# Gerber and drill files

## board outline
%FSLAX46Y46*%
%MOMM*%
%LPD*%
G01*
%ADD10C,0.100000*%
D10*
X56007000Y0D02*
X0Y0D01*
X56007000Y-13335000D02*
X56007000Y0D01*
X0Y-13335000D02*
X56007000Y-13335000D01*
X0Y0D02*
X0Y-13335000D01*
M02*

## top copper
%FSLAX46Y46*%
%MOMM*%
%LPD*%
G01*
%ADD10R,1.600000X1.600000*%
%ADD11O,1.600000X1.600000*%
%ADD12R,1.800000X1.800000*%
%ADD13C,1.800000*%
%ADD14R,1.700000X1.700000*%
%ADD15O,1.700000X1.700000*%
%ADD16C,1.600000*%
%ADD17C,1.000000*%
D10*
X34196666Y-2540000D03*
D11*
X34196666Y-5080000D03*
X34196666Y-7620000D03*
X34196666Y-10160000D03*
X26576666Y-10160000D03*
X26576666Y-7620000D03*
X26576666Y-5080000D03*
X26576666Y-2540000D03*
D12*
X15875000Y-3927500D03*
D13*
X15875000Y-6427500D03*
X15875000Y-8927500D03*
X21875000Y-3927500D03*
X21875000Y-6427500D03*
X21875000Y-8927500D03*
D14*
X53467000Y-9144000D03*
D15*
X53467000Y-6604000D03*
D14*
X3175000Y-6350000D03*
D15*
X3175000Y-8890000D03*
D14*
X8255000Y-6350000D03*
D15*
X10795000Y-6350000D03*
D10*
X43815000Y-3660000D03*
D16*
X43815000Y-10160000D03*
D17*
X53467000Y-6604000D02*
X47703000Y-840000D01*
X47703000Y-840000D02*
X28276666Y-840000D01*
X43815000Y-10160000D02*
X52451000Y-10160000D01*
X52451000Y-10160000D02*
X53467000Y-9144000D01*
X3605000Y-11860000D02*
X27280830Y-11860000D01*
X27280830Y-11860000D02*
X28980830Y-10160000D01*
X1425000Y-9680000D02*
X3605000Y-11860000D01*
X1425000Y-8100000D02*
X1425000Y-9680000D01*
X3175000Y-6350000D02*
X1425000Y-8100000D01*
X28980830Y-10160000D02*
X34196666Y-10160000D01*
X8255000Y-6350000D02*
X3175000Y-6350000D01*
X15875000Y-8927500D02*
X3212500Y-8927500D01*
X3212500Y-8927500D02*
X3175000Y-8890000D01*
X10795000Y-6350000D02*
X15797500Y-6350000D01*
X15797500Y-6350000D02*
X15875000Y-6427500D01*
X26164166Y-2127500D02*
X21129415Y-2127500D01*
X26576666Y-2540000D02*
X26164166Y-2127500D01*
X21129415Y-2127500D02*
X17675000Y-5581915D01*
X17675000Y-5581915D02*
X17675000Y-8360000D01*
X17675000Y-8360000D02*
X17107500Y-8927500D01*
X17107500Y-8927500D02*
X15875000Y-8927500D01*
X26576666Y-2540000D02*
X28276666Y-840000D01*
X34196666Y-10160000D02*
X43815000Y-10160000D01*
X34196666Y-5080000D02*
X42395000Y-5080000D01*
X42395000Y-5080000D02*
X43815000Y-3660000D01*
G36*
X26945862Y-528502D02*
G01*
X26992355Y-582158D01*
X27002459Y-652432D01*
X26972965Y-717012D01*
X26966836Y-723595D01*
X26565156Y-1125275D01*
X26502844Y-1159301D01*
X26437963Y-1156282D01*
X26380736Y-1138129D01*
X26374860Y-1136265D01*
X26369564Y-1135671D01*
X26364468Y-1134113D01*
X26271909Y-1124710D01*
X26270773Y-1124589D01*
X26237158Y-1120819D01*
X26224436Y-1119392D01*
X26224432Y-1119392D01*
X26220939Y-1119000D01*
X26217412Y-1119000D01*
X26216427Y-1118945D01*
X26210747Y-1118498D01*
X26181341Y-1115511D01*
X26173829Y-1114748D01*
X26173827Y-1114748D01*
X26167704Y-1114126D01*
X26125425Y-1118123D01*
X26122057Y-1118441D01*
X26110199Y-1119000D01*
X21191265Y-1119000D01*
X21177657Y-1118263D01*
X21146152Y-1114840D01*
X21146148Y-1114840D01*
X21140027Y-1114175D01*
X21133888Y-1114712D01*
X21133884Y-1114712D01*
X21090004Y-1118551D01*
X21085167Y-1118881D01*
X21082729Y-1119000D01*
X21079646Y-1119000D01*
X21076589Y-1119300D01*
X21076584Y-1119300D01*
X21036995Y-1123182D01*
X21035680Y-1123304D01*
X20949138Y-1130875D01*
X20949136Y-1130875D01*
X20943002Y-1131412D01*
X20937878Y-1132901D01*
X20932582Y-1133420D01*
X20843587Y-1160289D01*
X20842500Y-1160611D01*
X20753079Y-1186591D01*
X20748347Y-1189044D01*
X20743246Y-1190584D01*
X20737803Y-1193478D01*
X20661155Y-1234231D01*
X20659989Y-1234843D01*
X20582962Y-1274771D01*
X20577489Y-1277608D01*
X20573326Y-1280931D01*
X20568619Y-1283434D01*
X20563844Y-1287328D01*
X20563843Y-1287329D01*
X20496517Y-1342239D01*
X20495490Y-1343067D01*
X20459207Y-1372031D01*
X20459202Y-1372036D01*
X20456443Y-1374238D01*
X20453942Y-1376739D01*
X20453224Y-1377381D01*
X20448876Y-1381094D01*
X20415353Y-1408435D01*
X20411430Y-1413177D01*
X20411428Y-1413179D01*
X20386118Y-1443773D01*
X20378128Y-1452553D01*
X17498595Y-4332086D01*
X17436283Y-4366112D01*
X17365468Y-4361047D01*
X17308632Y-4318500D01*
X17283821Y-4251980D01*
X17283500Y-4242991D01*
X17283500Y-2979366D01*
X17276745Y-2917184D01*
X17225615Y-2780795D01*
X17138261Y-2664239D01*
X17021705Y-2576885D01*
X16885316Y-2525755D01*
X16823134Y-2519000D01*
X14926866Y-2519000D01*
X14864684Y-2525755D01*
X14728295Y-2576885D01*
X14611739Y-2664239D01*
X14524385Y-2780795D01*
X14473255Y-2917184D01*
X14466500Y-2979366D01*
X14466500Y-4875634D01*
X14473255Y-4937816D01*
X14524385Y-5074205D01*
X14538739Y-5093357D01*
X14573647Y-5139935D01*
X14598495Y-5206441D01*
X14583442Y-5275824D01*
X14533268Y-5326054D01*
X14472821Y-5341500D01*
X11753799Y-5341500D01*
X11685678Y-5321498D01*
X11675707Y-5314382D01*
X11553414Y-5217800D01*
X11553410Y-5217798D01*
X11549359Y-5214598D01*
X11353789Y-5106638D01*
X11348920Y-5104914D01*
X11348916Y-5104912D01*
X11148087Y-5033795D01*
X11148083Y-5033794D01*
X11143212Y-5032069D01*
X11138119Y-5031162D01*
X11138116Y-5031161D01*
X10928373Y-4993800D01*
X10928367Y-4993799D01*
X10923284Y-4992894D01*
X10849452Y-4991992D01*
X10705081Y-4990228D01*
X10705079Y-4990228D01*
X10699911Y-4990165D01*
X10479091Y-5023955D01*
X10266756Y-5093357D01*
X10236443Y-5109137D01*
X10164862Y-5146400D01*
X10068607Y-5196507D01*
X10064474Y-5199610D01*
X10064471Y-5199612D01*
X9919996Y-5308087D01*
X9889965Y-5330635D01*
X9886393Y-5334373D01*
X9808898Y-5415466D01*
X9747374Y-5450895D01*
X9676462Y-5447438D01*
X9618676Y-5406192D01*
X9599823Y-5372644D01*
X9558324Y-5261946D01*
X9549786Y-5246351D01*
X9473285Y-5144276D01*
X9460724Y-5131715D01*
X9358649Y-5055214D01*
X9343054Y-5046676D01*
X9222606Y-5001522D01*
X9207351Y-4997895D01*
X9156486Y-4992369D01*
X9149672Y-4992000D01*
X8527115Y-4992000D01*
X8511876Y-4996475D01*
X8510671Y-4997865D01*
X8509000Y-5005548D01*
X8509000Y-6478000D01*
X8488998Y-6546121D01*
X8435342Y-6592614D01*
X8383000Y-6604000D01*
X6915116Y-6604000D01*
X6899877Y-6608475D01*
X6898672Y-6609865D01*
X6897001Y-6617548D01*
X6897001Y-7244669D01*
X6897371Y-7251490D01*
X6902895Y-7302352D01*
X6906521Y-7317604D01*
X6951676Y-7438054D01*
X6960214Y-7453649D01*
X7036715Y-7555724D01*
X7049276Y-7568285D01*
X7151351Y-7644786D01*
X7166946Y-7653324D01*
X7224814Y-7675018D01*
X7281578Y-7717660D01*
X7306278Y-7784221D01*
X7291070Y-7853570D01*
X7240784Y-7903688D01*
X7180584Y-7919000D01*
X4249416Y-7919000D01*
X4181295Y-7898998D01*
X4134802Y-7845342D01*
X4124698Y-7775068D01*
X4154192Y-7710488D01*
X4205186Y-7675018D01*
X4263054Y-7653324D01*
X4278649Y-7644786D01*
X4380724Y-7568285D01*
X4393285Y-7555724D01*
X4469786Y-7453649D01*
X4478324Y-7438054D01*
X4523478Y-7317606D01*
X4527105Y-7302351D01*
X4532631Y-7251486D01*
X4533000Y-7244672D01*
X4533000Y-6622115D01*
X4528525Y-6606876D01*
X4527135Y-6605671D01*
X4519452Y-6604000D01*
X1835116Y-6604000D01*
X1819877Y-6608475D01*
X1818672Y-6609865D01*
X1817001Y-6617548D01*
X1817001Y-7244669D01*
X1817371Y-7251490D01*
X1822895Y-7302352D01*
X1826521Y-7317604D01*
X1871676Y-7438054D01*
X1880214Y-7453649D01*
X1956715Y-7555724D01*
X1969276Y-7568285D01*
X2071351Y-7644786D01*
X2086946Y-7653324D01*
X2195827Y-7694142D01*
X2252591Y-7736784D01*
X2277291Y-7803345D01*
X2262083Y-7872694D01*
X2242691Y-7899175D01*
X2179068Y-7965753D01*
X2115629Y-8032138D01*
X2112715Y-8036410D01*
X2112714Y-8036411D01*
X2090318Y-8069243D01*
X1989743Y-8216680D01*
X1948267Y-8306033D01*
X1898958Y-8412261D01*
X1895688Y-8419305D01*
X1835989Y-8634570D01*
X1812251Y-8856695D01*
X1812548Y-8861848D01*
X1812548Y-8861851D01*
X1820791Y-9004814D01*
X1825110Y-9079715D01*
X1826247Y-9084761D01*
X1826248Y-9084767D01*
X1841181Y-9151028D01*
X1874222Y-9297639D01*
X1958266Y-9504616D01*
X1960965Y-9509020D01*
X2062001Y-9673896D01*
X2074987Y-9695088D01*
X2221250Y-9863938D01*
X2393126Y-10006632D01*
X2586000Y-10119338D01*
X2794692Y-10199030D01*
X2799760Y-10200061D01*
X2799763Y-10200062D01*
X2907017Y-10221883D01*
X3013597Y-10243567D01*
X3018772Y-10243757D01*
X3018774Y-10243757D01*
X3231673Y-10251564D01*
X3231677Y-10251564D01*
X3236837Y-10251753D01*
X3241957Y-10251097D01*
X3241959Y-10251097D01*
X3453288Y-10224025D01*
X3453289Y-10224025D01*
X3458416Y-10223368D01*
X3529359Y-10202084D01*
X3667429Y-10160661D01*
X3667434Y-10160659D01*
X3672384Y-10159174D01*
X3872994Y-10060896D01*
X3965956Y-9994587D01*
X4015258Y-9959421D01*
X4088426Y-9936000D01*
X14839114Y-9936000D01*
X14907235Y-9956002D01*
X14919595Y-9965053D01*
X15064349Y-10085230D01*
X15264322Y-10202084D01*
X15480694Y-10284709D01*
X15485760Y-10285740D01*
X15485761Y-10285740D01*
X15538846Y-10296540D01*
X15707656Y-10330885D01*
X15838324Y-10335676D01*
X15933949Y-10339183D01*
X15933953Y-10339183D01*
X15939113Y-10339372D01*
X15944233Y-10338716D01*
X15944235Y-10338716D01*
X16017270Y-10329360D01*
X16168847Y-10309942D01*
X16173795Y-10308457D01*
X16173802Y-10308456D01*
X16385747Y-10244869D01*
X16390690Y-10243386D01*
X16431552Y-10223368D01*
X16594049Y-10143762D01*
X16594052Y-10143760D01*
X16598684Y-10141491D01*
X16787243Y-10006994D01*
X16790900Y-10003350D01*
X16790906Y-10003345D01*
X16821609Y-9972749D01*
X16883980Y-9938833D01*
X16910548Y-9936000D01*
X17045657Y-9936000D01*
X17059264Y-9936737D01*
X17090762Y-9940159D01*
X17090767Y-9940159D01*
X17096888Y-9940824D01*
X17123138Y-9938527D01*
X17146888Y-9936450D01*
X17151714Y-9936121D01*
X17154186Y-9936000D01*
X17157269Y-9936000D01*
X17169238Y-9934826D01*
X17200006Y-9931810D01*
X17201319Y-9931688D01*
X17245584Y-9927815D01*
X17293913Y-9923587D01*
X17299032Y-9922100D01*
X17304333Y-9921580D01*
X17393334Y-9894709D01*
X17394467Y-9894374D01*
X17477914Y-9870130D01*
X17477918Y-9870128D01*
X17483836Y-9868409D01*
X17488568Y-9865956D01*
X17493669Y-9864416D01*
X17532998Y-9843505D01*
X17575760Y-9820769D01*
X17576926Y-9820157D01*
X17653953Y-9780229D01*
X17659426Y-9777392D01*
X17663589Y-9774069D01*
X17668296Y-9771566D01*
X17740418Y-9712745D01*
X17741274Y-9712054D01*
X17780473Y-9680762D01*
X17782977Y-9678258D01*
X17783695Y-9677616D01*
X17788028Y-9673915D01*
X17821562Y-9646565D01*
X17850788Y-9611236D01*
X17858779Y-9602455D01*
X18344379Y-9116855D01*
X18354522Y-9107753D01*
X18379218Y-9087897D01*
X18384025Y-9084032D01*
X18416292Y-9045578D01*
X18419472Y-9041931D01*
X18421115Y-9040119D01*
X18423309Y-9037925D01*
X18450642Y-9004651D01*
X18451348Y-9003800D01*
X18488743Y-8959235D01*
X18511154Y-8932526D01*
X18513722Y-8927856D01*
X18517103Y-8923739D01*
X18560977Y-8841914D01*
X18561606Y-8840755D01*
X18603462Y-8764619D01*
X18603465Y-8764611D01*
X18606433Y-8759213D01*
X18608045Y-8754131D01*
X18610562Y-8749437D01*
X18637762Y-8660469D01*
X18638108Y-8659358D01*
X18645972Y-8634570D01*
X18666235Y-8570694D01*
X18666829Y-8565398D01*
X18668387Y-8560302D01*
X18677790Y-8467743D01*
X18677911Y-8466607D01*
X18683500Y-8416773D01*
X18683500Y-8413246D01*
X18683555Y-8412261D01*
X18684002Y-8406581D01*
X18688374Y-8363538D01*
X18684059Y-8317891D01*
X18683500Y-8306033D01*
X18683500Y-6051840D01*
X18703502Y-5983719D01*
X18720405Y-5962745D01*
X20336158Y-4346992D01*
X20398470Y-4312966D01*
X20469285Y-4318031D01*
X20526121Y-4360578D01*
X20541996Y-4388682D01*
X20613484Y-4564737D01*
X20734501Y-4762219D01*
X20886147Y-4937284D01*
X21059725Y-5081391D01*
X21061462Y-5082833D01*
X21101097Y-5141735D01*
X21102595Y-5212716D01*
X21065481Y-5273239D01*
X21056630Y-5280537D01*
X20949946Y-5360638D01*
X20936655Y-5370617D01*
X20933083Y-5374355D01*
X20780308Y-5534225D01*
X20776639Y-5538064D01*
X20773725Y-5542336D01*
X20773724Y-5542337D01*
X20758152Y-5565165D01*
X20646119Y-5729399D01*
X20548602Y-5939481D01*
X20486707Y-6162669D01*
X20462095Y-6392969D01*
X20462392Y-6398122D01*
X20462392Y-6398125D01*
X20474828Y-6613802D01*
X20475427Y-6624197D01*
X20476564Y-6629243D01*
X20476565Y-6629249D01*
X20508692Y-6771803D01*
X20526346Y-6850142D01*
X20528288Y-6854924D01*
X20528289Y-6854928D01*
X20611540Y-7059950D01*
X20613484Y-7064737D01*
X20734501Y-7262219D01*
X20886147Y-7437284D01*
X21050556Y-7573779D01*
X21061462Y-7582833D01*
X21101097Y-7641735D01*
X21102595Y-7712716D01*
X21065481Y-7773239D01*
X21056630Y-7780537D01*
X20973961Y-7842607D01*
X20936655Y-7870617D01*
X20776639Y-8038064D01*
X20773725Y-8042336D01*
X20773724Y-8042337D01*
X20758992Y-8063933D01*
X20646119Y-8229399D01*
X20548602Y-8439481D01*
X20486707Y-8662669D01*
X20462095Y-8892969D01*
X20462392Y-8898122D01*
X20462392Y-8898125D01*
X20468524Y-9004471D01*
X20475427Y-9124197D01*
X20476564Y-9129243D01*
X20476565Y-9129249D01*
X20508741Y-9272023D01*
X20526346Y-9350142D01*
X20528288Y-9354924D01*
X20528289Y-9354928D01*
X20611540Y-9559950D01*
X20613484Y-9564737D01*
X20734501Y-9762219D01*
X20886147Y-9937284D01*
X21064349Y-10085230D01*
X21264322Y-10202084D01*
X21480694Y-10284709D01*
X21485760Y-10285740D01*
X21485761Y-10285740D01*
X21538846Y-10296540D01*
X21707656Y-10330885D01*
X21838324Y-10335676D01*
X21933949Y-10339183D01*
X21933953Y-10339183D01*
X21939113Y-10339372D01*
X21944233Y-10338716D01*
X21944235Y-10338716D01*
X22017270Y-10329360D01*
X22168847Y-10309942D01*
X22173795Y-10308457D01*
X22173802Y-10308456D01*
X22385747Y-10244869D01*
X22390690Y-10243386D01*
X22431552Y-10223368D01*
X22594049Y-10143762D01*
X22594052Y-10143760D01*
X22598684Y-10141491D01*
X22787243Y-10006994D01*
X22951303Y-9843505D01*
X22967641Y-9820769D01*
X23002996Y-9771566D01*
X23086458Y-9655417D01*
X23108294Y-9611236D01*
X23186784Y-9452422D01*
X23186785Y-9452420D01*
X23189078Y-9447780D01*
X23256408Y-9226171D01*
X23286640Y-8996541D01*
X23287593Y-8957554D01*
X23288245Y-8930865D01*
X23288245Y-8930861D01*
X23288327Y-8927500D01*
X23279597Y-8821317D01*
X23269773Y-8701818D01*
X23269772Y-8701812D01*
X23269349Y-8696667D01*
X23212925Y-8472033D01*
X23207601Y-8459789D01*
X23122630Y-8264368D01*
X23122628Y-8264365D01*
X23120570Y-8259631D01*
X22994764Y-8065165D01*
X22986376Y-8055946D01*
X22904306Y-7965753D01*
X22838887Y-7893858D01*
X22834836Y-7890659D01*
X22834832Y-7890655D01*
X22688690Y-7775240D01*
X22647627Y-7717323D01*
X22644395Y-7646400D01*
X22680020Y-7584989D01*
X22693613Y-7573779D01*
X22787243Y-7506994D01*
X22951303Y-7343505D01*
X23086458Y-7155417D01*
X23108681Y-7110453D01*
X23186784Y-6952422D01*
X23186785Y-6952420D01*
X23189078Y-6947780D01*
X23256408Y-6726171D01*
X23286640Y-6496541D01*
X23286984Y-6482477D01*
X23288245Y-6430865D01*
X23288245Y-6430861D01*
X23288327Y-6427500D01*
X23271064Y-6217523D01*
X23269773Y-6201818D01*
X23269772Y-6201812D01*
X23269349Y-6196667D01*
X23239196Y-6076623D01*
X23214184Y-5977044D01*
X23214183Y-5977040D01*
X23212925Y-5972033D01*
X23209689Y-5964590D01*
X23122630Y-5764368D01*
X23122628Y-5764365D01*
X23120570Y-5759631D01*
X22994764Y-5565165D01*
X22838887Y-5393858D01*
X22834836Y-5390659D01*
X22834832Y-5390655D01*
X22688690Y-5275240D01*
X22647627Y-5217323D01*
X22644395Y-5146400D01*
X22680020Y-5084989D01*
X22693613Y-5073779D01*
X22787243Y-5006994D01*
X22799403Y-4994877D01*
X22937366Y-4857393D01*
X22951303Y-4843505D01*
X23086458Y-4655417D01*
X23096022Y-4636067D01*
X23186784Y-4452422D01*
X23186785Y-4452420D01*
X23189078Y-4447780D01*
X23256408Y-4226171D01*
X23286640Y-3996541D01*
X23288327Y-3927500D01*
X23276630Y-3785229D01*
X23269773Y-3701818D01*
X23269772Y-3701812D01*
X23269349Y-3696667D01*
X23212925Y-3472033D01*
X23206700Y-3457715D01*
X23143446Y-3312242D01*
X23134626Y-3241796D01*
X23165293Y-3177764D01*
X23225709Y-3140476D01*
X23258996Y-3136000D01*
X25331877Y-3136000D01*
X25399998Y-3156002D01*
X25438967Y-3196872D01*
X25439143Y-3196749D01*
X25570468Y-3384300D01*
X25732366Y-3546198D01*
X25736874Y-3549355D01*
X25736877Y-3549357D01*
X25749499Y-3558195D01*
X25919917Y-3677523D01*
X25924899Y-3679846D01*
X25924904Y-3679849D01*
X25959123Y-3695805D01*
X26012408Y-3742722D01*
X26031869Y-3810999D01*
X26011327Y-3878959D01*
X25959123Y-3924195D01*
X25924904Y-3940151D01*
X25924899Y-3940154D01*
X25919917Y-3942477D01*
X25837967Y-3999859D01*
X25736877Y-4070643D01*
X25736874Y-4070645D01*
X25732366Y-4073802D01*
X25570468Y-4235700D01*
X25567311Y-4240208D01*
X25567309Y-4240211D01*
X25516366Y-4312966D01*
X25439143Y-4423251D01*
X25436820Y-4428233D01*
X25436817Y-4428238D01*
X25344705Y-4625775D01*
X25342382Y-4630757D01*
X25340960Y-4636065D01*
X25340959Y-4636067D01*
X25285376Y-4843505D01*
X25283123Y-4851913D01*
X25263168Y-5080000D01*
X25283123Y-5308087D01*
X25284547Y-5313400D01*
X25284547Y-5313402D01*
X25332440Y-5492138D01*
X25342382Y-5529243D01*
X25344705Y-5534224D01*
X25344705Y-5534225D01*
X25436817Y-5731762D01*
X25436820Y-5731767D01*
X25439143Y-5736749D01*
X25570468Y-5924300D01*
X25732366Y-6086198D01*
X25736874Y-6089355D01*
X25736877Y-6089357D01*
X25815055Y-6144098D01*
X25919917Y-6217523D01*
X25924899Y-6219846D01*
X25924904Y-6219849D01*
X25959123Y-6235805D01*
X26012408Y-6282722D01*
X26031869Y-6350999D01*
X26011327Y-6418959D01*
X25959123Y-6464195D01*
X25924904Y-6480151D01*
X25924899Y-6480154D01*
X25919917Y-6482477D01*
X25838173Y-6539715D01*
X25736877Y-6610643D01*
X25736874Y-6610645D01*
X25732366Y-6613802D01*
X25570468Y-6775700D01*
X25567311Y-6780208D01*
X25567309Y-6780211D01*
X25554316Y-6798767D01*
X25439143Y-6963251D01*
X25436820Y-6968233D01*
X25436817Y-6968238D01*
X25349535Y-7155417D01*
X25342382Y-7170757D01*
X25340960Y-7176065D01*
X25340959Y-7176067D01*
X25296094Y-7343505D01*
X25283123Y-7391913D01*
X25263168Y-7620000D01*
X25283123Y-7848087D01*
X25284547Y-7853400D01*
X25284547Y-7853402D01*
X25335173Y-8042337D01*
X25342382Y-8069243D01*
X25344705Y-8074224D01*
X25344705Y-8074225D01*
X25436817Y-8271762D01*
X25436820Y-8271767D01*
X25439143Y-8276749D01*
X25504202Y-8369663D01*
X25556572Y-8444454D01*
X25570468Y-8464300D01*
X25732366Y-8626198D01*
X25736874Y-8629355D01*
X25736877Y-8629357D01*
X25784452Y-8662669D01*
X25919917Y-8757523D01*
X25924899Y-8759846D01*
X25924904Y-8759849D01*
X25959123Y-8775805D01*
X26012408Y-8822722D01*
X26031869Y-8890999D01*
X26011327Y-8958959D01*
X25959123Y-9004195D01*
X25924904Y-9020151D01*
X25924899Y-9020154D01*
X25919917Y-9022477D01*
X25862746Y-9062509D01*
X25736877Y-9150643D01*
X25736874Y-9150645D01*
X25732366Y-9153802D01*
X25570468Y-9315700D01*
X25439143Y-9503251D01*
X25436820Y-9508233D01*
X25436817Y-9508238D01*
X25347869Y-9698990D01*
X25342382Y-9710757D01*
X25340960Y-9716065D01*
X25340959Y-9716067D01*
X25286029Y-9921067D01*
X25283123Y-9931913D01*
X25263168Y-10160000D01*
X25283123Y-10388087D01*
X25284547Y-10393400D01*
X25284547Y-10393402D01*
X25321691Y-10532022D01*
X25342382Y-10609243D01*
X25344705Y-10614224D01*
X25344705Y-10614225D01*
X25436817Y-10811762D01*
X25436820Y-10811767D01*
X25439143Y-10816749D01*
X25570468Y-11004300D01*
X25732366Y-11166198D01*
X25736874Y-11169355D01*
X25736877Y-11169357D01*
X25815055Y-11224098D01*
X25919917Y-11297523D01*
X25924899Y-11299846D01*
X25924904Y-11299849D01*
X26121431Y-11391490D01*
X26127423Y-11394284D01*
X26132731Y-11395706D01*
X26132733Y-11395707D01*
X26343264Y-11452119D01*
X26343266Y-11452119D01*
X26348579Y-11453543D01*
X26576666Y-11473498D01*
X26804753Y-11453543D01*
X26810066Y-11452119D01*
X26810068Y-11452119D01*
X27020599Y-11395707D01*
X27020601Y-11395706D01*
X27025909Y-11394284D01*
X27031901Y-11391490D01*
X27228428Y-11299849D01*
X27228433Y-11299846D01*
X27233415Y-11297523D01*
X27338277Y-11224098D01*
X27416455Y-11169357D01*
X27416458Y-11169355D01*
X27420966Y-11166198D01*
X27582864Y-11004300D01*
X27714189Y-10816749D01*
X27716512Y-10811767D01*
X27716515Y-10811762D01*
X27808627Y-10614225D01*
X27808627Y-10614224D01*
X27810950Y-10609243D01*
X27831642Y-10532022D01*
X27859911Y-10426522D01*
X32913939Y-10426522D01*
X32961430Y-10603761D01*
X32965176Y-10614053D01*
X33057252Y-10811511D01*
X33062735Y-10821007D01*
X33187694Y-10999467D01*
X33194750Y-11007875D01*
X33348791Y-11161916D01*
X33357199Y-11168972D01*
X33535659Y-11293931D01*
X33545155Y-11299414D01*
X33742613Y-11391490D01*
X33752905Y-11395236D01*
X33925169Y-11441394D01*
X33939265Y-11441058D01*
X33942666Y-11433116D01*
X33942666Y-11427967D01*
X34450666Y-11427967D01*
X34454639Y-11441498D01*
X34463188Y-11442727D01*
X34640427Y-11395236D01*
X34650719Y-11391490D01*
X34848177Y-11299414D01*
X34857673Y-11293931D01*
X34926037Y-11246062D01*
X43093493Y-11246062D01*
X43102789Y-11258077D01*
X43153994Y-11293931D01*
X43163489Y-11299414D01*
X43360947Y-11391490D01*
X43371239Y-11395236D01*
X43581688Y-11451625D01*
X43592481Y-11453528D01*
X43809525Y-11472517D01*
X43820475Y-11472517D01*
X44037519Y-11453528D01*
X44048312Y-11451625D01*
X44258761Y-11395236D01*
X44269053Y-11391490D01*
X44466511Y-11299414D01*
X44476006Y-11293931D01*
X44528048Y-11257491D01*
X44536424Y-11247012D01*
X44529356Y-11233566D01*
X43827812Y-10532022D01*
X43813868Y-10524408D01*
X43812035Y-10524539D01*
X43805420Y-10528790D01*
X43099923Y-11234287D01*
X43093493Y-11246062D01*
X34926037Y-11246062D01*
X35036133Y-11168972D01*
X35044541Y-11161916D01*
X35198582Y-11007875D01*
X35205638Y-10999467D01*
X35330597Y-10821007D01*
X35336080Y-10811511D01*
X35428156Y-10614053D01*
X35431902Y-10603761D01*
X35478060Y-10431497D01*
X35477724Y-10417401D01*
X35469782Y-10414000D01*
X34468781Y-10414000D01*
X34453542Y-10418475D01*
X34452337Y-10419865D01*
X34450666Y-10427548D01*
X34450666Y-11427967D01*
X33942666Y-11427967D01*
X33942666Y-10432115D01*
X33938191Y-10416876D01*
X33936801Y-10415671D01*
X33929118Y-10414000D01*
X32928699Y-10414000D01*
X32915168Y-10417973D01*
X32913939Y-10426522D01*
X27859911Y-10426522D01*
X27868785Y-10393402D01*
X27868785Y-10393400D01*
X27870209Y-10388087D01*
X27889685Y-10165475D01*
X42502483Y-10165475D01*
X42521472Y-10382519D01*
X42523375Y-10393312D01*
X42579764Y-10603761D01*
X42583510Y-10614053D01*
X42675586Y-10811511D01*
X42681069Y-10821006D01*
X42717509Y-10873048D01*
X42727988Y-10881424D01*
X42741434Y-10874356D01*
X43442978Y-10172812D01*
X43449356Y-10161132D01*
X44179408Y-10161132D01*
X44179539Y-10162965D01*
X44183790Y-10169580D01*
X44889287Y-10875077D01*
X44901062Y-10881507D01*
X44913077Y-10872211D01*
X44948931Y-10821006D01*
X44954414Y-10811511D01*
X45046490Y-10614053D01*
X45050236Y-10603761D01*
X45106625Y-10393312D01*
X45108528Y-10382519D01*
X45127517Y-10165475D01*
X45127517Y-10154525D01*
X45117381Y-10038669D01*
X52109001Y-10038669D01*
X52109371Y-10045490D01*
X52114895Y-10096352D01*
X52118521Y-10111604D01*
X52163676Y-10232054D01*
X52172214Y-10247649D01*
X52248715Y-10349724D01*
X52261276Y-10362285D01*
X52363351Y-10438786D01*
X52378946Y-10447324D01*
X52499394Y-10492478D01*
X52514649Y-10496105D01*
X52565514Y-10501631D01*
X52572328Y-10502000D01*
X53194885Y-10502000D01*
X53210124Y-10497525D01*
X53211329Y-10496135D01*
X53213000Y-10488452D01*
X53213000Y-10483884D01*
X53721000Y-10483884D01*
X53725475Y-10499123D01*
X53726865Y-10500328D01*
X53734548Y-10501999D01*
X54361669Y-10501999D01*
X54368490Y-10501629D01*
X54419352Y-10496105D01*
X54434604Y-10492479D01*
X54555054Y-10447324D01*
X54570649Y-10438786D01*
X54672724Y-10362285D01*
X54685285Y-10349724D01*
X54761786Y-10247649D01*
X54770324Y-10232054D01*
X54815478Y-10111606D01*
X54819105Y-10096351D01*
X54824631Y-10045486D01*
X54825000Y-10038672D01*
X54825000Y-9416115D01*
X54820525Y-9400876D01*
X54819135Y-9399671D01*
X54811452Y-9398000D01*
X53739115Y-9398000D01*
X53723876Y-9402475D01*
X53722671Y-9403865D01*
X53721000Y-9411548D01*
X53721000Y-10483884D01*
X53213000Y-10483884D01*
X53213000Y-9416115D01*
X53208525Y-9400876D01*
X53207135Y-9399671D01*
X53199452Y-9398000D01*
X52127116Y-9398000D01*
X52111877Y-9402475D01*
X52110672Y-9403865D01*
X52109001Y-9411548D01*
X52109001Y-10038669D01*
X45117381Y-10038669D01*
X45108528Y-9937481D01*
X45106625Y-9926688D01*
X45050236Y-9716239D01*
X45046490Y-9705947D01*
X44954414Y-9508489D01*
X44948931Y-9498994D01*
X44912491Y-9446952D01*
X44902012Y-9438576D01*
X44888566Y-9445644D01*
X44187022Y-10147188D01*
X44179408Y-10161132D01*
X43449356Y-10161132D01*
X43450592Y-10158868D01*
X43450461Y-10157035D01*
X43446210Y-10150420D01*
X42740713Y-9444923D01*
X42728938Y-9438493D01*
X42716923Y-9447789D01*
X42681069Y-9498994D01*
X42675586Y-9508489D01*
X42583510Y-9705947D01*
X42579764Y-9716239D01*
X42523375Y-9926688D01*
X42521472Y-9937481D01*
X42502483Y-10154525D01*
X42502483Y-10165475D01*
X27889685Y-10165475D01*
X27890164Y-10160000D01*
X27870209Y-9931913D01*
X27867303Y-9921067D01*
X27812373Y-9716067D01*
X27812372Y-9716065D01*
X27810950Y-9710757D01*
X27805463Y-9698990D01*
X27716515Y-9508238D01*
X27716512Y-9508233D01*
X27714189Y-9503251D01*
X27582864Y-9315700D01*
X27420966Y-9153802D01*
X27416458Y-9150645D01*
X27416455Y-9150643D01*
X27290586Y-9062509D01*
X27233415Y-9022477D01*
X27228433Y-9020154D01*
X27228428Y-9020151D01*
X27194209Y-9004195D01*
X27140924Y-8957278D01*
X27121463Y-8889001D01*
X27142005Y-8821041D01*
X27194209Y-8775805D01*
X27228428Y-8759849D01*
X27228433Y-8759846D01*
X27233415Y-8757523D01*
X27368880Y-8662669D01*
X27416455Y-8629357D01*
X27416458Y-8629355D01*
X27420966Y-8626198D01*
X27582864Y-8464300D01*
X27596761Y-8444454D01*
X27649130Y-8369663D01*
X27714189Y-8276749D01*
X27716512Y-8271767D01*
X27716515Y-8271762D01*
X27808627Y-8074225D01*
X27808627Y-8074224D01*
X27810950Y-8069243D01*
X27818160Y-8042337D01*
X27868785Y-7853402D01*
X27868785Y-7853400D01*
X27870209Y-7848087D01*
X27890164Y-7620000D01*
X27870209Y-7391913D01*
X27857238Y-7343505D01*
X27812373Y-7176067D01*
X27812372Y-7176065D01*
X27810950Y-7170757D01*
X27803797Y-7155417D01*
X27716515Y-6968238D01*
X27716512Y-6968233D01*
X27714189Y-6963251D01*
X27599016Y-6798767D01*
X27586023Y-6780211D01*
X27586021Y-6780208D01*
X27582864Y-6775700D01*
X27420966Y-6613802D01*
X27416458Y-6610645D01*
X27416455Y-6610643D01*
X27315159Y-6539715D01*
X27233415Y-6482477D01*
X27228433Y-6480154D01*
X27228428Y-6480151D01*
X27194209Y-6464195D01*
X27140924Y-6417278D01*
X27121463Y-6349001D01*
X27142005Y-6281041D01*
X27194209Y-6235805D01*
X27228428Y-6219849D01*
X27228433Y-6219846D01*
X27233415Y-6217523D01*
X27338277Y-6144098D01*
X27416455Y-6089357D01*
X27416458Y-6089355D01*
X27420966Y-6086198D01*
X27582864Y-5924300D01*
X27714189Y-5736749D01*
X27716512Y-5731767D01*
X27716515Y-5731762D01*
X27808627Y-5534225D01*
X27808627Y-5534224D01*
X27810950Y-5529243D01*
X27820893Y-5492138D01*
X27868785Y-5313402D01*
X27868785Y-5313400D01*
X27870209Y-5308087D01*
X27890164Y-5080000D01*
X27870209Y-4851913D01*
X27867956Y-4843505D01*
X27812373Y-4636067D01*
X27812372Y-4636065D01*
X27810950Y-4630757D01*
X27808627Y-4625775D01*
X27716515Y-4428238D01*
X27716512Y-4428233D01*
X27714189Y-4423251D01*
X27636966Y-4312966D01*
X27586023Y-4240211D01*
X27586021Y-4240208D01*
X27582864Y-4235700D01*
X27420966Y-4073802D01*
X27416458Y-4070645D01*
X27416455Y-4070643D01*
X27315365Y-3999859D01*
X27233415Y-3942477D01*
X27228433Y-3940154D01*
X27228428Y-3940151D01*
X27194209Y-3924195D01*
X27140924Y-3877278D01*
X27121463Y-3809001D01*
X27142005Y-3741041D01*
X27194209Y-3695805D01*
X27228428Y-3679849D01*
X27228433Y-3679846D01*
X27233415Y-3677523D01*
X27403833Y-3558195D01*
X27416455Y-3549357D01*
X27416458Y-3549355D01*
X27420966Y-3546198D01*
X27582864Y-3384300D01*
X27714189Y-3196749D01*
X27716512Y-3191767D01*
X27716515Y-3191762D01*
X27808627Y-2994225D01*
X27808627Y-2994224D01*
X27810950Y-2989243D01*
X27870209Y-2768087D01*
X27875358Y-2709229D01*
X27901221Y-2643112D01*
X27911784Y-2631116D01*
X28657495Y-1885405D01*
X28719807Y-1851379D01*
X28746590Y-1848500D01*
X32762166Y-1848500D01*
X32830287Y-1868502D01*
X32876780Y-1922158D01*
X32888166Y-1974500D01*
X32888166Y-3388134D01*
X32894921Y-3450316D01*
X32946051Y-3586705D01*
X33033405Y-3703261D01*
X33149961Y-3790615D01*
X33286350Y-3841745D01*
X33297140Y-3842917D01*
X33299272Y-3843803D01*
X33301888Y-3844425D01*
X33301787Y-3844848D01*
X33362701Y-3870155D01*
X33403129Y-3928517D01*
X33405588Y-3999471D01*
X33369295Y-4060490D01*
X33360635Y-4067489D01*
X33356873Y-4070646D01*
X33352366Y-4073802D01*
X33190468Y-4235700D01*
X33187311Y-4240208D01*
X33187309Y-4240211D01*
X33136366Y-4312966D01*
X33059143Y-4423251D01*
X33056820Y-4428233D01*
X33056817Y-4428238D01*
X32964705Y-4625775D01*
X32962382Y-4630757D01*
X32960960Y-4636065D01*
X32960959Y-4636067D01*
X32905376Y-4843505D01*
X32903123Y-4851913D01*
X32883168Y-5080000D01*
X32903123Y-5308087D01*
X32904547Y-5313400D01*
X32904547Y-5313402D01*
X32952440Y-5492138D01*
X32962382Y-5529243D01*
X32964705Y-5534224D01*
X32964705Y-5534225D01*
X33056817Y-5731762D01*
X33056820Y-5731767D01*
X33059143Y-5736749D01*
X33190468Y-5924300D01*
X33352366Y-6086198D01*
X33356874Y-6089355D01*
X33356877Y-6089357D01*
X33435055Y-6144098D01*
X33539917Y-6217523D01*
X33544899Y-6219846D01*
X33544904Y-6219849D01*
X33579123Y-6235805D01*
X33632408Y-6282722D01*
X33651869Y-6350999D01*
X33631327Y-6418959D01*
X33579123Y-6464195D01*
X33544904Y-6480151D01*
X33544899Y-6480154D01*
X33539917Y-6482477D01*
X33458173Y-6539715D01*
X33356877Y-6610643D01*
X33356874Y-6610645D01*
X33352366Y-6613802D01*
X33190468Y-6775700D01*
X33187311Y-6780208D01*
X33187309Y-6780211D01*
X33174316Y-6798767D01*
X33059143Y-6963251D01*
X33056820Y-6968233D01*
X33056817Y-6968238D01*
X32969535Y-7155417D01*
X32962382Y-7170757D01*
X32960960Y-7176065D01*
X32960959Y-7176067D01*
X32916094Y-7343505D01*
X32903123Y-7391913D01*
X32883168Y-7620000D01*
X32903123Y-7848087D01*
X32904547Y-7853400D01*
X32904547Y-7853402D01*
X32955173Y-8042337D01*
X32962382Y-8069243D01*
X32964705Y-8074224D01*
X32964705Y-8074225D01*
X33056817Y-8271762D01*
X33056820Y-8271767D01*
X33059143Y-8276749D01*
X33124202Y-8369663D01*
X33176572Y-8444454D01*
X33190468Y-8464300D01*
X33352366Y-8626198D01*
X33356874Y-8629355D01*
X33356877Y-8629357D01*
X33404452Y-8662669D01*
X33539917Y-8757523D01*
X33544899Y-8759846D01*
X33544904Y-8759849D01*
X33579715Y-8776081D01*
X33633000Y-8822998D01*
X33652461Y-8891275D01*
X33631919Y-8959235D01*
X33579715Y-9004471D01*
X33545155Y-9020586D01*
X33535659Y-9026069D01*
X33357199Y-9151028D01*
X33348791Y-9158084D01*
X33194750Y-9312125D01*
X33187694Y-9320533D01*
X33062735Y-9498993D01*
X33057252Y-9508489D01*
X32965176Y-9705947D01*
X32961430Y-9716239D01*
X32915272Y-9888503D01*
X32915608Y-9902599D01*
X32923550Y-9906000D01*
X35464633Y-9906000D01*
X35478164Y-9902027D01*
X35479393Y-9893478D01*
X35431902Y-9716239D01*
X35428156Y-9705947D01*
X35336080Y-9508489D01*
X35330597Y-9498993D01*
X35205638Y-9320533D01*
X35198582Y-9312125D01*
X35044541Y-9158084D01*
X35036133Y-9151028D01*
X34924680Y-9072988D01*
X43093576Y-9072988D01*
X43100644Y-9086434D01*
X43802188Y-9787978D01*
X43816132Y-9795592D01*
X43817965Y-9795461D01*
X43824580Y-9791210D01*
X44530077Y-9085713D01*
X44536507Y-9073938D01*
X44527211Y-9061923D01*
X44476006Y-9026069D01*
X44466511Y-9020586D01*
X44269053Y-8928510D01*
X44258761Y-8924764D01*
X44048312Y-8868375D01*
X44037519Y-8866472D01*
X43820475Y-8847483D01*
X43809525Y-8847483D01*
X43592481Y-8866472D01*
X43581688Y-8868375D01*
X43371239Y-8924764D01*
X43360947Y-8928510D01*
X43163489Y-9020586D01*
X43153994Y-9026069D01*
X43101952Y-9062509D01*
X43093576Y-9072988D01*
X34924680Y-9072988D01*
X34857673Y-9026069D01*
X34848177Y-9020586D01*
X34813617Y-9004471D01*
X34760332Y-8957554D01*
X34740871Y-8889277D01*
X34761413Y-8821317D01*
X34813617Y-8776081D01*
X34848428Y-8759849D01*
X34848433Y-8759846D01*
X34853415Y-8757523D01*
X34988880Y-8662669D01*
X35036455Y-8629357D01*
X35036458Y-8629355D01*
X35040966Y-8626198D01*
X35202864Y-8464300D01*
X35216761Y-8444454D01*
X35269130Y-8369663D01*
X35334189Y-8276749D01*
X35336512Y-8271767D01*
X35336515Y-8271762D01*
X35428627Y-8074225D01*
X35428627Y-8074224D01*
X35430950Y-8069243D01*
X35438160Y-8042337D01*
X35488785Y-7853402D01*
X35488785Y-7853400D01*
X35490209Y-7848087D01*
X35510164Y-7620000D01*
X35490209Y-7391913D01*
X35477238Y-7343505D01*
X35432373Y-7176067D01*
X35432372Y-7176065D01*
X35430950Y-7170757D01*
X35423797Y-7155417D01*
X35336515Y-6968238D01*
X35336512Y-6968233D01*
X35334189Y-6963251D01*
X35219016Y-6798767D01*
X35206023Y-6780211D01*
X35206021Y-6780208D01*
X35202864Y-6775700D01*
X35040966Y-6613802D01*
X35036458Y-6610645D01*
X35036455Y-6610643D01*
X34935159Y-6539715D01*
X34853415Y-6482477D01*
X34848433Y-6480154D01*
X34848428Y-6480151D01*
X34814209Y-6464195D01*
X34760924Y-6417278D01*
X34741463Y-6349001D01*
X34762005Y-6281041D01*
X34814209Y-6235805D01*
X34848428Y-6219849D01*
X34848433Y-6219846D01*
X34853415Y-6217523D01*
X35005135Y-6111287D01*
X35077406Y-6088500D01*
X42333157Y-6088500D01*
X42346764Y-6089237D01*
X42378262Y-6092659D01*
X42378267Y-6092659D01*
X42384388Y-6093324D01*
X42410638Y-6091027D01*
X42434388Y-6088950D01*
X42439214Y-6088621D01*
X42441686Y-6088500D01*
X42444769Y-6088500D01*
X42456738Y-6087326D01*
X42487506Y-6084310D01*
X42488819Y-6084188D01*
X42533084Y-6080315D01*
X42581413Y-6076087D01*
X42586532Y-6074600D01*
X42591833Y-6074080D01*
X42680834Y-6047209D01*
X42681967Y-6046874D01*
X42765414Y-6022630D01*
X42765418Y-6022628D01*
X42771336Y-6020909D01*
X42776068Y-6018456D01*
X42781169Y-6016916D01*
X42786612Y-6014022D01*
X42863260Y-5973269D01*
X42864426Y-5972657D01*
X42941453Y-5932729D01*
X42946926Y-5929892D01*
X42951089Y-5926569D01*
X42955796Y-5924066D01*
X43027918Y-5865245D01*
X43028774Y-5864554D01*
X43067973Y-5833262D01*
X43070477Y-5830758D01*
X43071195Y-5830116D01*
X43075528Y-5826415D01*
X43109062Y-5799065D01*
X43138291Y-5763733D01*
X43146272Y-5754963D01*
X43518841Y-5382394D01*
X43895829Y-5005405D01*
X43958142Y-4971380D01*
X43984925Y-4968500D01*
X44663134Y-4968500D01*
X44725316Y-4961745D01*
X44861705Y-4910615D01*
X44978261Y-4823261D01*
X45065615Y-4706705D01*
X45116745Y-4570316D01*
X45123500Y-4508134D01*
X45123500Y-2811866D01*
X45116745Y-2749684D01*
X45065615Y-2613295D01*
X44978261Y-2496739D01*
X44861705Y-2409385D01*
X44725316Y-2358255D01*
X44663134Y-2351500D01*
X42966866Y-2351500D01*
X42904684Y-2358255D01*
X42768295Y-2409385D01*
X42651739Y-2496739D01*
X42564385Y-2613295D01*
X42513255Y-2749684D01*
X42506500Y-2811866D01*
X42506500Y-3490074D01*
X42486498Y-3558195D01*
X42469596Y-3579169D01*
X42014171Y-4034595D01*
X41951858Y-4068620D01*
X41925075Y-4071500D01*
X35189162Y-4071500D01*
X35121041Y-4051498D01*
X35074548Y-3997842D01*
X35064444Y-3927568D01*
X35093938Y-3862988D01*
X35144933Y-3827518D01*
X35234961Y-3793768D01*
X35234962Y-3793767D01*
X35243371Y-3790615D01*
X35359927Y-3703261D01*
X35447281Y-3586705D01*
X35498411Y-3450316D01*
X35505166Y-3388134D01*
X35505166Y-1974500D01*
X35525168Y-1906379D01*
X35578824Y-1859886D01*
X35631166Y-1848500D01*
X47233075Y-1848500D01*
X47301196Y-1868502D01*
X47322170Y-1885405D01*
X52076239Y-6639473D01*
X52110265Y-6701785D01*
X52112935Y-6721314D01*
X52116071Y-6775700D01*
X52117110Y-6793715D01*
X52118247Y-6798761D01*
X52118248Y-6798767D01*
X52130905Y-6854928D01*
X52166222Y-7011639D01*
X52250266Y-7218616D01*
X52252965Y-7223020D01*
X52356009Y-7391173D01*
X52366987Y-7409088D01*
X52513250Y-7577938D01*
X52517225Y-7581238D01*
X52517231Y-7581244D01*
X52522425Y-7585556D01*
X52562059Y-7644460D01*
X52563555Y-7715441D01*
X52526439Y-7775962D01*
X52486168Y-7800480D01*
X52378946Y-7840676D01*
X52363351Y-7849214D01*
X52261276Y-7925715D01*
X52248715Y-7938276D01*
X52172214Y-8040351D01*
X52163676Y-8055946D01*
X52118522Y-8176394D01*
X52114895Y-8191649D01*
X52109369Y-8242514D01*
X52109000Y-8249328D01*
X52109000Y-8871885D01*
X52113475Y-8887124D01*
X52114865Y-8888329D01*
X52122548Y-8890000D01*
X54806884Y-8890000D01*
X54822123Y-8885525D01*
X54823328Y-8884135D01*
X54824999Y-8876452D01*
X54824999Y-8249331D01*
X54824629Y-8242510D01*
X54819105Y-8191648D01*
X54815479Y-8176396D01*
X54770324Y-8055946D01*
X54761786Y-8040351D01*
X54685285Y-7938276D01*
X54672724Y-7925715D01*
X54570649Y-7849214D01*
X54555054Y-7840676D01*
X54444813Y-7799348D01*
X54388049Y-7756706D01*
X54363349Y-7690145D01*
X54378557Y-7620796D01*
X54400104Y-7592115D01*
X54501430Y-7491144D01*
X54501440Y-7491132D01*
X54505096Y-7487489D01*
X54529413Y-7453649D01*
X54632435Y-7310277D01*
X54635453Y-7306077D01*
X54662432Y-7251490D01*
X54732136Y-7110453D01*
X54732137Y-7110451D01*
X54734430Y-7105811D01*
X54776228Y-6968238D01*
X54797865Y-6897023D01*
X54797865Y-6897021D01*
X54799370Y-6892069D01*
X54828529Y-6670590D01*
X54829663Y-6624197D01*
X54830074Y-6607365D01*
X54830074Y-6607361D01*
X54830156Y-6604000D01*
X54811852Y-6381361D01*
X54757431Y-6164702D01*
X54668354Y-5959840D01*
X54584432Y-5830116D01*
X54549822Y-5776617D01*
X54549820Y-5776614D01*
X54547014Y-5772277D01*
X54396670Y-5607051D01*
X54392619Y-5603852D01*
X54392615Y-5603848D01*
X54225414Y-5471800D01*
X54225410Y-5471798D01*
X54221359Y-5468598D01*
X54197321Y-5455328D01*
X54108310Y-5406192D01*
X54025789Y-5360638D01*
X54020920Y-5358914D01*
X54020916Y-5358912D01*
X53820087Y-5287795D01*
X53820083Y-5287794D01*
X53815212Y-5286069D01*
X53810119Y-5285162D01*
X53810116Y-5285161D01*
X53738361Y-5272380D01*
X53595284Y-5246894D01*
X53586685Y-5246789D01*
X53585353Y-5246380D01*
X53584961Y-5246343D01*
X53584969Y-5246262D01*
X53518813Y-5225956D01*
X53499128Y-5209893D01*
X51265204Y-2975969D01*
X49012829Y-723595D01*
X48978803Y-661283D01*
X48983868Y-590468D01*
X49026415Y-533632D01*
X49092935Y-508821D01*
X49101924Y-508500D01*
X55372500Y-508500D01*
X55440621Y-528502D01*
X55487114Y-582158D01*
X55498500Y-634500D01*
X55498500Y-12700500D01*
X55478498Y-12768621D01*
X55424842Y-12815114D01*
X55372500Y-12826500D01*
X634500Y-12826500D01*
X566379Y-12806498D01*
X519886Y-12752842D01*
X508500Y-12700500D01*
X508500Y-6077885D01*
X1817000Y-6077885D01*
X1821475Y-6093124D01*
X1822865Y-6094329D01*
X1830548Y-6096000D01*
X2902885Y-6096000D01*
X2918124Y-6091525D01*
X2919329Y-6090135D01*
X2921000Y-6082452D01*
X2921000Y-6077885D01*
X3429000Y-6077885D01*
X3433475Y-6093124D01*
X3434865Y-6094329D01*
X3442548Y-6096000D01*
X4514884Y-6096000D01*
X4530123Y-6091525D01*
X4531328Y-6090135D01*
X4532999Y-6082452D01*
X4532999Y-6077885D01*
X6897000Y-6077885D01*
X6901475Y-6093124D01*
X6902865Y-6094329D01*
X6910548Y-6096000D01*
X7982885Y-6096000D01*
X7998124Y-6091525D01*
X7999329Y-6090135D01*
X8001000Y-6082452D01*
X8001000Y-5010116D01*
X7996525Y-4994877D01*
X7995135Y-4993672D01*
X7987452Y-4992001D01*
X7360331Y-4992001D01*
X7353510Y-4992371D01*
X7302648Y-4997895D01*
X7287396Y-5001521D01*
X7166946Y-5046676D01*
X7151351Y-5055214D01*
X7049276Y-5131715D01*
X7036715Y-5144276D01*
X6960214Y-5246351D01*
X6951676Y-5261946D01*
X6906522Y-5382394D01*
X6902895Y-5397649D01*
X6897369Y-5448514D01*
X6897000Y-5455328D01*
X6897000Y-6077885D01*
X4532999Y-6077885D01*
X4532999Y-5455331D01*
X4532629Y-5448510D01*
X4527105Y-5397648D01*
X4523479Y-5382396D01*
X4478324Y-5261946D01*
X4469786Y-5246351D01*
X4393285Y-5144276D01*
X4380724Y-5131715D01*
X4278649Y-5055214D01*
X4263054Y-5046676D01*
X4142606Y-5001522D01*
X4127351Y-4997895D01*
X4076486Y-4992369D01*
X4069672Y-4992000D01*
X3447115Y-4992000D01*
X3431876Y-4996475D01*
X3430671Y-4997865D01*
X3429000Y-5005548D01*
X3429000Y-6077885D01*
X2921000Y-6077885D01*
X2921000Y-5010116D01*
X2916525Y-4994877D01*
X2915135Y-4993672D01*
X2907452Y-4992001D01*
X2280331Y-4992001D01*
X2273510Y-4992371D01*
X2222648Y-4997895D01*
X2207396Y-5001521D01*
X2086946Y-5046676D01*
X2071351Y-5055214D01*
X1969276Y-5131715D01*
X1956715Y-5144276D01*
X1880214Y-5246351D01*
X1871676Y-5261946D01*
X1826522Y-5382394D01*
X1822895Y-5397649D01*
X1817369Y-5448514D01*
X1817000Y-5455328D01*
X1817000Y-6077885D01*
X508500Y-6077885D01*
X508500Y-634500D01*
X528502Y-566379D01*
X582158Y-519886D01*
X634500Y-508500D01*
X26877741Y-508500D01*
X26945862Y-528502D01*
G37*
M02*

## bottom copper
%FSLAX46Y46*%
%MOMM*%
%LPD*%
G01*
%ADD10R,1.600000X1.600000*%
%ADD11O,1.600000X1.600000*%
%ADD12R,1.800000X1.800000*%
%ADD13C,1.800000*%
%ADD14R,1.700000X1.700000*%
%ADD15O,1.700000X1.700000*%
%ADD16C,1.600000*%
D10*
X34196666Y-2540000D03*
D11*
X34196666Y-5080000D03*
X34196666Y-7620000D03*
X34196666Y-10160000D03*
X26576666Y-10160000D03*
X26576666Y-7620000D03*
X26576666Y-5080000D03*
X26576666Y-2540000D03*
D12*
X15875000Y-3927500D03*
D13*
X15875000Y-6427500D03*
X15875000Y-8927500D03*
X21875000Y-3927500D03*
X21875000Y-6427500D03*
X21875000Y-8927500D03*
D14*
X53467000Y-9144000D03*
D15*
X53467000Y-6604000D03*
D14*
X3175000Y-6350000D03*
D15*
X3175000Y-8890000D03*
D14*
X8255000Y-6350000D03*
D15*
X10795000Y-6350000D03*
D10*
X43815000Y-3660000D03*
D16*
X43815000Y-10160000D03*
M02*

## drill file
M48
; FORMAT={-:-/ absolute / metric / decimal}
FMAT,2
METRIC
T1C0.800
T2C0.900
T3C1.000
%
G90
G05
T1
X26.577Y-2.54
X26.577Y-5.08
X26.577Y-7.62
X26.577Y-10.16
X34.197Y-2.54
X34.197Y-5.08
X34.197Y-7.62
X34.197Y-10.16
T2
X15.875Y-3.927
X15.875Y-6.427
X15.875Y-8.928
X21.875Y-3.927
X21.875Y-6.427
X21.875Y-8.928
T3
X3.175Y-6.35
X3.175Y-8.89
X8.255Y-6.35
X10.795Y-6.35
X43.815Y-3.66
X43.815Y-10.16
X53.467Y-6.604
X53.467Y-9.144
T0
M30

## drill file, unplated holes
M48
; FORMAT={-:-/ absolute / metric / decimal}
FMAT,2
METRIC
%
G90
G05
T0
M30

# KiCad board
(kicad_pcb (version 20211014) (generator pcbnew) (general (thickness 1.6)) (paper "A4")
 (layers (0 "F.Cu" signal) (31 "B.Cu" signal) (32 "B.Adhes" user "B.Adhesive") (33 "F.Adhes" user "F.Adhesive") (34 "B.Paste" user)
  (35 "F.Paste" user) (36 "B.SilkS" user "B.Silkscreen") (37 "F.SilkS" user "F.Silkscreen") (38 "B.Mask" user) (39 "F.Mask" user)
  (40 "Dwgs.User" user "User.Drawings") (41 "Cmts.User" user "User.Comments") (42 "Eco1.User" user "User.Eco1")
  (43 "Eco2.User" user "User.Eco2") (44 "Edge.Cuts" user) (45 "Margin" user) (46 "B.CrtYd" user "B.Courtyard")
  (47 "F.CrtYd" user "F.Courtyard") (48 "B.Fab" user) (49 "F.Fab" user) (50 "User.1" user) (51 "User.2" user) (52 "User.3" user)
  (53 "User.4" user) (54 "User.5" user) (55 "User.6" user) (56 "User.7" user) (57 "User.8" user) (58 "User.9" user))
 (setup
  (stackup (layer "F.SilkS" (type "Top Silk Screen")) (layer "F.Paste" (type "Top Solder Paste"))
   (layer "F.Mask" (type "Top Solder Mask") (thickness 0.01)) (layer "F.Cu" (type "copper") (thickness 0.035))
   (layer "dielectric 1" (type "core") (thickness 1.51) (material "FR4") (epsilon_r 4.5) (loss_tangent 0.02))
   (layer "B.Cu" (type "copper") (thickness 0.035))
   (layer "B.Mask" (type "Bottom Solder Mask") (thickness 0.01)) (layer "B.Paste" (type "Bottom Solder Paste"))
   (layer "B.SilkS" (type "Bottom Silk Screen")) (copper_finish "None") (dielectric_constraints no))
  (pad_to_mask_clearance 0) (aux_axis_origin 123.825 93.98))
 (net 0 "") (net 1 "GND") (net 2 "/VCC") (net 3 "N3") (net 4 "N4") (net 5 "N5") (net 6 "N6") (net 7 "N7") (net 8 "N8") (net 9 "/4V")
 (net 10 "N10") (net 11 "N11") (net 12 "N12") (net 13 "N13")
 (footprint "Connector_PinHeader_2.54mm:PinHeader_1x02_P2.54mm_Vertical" (layer "B.Cu") (at 127 100.33 180)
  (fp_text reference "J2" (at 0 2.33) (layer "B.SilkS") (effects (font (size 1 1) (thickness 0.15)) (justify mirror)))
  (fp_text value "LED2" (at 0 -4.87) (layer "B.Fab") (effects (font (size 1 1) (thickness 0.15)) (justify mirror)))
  (pad "1" thru_hole rect (at 0 0 180) (size 1.7 1.7) (drill 1) (layers *.Cu *.Mask) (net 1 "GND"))
  (pad "2" thru_hole oval (at 0 -2.54 180) (size 1.7 1.7) (drill 1) (layers *.Cu *.Mask) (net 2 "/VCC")))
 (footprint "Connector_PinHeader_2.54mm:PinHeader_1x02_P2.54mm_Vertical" (layer "B.Cu") (at 177.292 103.124)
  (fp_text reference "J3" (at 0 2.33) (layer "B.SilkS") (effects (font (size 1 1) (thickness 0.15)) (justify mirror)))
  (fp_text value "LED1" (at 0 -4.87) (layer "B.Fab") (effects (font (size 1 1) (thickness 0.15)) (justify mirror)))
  (pad "1" thru_hole rect (at 0 0) (size 1.7 1.7) (drill 1) (layers *.Cu *.Mask) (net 1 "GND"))
  (pad "2" thru_hole oval (at 0 -2.54) (size 1.7 1.7) (drill 1) (layers *.Cu *.Mask) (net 2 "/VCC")))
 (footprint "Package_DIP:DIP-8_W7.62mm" (layer "B.Cu") (at 158.021666 96.52 180)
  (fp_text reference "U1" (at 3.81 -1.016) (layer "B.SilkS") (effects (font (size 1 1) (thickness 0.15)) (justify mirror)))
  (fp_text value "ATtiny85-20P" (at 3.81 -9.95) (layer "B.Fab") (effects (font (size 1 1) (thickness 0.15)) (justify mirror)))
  (pad "1" thru_hole rect (at 0 0 180) (size 1.6 1.6) (drill 0.8) (layers *.Cu *.Mask) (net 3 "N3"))
  (pad "2" thru_hole oval (at 0 -2.54 180) (size 1.6 1.6) (drill 0.8) (layers *.Cu *.Mask) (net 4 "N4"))
  (pad "3" thru_hole oval (at 0 -5.08 180) (size 1.6 1.6) (drill 0.8) (layers *.Cu *.Mask) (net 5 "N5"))
  (pad "4" thru_hole oval (at 0 -7.62 180) (size 1.6 1.6) (drill 0.8) (layers *.Cu *.Mask) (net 1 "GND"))
  (pad "5" thru_hole oval (at 7.62 -7.62 180) (size 1.6 1.6) (drill 0.8) (layers *.Cu *.Mask) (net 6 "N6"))
  (pad "6" thru_hole oval (at 7.62 -5.08 180) (size 1.6 1.6) (drill 0.8) (layers *.Cu *.Mask) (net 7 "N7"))
  (pad "7" thru_hole oval (at 7.62 -2.54 180) (size 1.6 1.6) (drill 0.8) (layers *.Cu *.Mask) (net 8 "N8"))
  (pad "8" thru_hole oval (at 7.62 0 180) (size 1.6 1.6) (drill 0.8) (layers *.Cu *.Mask) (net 2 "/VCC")))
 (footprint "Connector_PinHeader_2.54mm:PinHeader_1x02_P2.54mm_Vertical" (layer "B.Cu") (at 132.08 100.33 -90)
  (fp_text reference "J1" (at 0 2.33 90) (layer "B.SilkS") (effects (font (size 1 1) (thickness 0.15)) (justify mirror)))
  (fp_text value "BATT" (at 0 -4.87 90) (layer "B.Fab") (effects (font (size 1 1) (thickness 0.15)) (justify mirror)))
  (pad "1" thru_hole rect (at 0 0 270) (size 1.7 1.7) (drill 1) (layers *.Cu *.Mask) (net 1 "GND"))
  (pad "2" thru_hole oval (at 0 -2.54 270) (size 1.7 1.7) (drill 1) (layers *.Cu *.Mask) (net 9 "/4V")))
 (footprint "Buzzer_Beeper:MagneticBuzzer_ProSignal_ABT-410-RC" (layer "B.Cu") (at 167.64 97.64 -90)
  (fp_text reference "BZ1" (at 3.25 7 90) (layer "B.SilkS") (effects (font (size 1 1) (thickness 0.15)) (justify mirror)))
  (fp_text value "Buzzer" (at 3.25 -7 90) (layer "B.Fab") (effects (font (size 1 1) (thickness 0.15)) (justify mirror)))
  (pad "1" thru_hole rect (at 0 0 270) (size 1.6 1.6) (drill 1) (layers *.Cu *.Mask) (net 4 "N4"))
  (pad "2" thru_hole circle (at 6.5 0 270) (size 1.6 1.6) (drill 1) (layers *.Cu *.Mask) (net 1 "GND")))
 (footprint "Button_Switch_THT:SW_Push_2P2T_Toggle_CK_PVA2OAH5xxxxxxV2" (layer "B.Cu") (at 139.7 97.9075 -90)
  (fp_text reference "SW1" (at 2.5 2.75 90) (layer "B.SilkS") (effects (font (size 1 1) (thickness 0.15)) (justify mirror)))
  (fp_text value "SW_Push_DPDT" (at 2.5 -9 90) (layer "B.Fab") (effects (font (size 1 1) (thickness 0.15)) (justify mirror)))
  (pad "1" thru_hole rect (at 0 0 270) (size 1.8 1.8) (drill 0.9) (layers *.Cu *.Mask) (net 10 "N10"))
  (pad "2" thru_hole circle (at 2.5 0 270) (size 1.8 1.8) (drill 0.9) (layers *.Cu *.Mask) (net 9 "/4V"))
  (pad "3" thru_hole circle (at 5 0 270) (size 1.8 1.8) (drill 0.9) (layers *.Cu *.Mask) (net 2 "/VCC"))
  (pad "4" thru_hole circle (at 0 -6 270) (size 1.8 1.8) (drill 0.9) (layers *.Cu *.Mask) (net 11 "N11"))
  (pad "5" thru_hole circle (at 2.5 -6 270) (size 1.8 1.8) (drill 0.9) (layers *.Cu *.Mask) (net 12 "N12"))
  (pad "6" thru_hole circle (at 5 -6 270) (size 1.8 1.8) (drill 0.9) (layers *.Cu *.Mask) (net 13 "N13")))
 (gr_line (start 123.825 93.98) (end 123.825 107.315) (layer "Edge.Cuts") (width 0.1))
 (gr_line (start 179.832 93.98) (end 123.825 93.98) (layer "Edge.Cuts") (width 0.1))
 (gr_line (start 123.825 107.315) (end 179.832 107.315) (layer "Edge.Cuts") (width 0.1))
 (gr_line (start 179.832 107.315) (end 179.832 93.98) (layer "Edge.Cuts") (width 0.1))
 (segment (start 166.22 99.06) (end 167.64 97.64) (width 1) (layer "F.Cu") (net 4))
 (segment (start 158.021666 99.06) (end 166.22 99.06) (width 1) (layer "F.Cu") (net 4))
 (segment (start 176.276 104.14) (end 177.292 103.124) (width 1) (layer "F.Cu") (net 1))
 (segment (start 127.43 105.84) (end 151.10583 105.84) (width 1) (layer "F.Cu") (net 1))
 (segment (start 152.80583 104.14) (end 158.021666 104.14) (width 1) (layer "F.Cu") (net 1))
 (segment (start 132.08 100.33) (end 127 100.33) (width 1) (layer "F.Cu") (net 1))
 (segment (start 158.021666 104.14) (end 167.64 104.14) (width 1) (layer "F.Cu") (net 1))
 (segment (start 151.10583 105.84) (end 152.80583 104.14) (width 1) (layer "F.Cu") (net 1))
 (segment (start 125.25 102.08) (end 125.25 103.66) (width 1) (layer "F.Cu") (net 1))
 (segment (start 125.25 103.66) (end 127.43 105.84) (width 1) (layer "F.Cu") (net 1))
 (segment (start 127 100.33) (end 125.25 102.08) (width 1) (layer "F.Cu") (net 1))
 (segment (start 167.64 104.14) (end 176.276 104.14) (width 1) (layer "F.Cu") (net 1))
 (segment (start 139.6225 100.33) (end 139.7 100.4075) (width 1) (layer "F.Cu") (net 9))
 (segment (start 134.62 100.33) (end 139.6225 100.33) (width 1) (layer "F.Cu") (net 9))
 (segment (start 150.401666 96.52) (end 152.101666 94.82) (width 1) (layer "F.Cu") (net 2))
 (segment (start 139.7 102.9075) (end 127.0375 102.9075) (width 1) (layer "F.Cu") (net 2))
 (segment (start 149.989166 96.1075) (end 144.954415 96.1075) (width 1) (layer "F.Cu") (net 2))
 (segment (start 140.9325 102.9075) (end 139.7 102.9075) (width 1) (layer "F.Cu") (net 2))
 (segment (start 150.401666 96.52) (end 149.989166 96.1075) (width 1) (layer "F.Cu") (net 2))
 (segment (start 141.5 99.561915) (end 141.5 102.34) (width 1) (layer "F.Cu") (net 2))
 (segment (start 144.954415 96.1075) (end 141.5 99.561915) (width 1) (layer "F.Cu") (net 2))
 (segment (start 177.292 100.584) (end 171.528 94.82) (width 1) (layer "F.Cu") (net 2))
 (segment (start 171.528 94.82) (end 152.101666 94.82) (width 1) (layer "F.Cu") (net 2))
 (segment (start 141.5 102.34) (end 140.9325 102.9075) (width 1) (layer "F.Cu") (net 2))
 (segment (start 127.0375 102.9075) (end 127 102.87) (width 1) (layer "F.Cu") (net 2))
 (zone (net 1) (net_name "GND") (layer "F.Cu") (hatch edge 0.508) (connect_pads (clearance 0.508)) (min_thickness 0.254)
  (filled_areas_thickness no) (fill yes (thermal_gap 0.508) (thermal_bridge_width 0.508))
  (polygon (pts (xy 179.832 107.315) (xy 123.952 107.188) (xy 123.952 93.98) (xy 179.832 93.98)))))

